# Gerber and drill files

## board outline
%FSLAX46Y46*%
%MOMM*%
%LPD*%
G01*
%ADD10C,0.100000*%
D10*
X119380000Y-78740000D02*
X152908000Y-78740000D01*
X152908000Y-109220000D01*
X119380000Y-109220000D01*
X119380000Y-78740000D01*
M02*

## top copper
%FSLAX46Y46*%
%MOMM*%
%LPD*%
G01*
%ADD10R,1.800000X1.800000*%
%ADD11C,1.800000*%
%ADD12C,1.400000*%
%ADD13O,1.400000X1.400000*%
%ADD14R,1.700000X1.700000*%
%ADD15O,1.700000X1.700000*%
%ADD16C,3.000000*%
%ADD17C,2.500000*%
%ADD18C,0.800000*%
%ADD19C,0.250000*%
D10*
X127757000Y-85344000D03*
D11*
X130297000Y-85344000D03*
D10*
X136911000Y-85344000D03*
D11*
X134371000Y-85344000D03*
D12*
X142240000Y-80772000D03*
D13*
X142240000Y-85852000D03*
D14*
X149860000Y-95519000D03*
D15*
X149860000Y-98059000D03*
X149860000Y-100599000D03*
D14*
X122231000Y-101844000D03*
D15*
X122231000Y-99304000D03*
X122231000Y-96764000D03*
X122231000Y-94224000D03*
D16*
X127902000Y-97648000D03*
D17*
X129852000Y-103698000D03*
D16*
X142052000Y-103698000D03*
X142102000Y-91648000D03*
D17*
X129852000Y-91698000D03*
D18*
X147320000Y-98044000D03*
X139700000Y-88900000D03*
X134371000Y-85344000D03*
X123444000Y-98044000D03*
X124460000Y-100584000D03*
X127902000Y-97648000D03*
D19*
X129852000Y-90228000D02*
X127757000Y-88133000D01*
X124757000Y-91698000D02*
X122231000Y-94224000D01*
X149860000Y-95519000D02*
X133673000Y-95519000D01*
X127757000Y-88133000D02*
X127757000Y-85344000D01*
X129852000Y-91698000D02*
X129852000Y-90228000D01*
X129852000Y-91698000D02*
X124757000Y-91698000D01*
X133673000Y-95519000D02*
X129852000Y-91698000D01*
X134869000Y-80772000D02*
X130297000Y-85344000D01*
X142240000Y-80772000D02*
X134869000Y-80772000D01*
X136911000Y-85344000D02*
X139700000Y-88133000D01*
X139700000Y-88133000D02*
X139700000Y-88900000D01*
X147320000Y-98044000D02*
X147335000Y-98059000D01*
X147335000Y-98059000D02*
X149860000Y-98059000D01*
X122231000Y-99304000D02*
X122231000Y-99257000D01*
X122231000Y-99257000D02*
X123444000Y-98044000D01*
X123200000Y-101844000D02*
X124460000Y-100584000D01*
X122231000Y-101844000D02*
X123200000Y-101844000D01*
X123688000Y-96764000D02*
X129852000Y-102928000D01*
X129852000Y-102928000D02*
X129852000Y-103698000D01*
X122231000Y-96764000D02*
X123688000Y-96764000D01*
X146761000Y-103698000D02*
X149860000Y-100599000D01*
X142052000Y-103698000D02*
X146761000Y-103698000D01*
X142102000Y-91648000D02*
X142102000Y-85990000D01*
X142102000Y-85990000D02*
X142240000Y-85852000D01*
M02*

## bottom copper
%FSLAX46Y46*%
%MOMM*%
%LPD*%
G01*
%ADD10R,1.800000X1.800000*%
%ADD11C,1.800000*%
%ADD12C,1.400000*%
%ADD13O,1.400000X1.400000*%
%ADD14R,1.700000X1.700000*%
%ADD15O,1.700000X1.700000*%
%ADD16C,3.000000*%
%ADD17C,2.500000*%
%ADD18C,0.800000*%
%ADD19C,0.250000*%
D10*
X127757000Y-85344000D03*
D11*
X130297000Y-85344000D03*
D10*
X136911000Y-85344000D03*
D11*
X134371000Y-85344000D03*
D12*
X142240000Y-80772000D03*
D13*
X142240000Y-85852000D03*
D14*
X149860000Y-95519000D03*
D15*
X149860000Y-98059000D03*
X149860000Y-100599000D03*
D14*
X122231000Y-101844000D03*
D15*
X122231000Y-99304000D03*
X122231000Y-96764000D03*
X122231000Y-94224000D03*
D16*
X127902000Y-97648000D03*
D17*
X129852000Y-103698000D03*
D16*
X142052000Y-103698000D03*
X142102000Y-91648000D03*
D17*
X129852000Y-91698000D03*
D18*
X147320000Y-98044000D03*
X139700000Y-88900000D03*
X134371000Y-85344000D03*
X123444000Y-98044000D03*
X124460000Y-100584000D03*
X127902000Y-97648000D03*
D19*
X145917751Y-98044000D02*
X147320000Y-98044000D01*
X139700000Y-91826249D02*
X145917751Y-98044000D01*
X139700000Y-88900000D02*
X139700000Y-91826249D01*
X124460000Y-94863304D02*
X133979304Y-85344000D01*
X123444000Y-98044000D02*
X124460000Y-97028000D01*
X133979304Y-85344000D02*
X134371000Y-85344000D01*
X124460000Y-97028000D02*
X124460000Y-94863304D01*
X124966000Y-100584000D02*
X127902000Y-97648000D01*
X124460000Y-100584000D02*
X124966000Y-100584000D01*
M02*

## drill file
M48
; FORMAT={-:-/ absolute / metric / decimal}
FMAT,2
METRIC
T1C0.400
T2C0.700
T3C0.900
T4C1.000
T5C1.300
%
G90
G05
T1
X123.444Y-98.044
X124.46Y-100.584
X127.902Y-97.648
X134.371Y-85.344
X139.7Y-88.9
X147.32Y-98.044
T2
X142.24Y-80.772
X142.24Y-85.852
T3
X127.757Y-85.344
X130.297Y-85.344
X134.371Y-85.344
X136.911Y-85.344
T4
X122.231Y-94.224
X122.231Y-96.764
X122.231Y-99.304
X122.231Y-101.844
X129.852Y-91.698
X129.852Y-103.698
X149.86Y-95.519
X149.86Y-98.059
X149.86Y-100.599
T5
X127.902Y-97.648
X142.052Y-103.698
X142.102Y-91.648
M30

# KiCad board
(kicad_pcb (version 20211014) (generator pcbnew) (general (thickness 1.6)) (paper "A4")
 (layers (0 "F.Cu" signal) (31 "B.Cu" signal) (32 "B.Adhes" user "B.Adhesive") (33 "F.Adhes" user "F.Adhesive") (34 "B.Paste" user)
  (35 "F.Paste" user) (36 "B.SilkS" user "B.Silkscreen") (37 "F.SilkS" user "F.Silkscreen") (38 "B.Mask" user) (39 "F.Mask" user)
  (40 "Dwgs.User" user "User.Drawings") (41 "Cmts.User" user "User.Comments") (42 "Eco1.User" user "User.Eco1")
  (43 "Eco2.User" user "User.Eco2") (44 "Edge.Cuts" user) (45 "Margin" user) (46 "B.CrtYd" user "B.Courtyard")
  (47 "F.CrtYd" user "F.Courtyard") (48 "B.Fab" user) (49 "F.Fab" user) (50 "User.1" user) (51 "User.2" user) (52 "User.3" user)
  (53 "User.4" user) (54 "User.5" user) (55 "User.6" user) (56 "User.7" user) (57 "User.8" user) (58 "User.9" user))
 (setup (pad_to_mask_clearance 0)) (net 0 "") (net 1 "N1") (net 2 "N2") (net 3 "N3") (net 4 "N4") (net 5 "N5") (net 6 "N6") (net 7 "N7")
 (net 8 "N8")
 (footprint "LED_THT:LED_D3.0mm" (layer "F.Cu") (at 127.757 85.344)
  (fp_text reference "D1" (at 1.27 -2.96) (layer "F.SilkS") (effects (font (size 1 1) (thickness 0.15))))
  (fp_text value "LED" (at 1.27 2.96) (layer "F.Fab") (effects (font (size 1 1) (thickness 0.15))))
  (pad "1" thru_hole rect (at 0 0) (size 1.8 1.8) (drill 0.9) (layers *.Cu *.Mask) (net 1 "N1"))
  (pad "2" thru_hole circle (at 2.54 0) (size 1.8 1.8) (drill 0.9) (layers *.Cu *.Mask) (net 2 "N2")))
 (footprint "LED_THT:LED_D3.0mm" (layer "F.Cu") (at 136.911 85.344 180)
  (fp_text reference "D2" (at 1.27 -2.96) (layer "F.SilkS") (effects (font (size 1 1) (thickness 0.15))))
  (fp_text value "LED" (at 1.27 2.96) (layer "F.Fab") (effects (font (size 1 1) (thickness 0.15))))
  (pad "1" thru_hole rect (at 0 0 180) (size 1.8 1.8) (drill 0.9) (layers *.Cu *.Mask) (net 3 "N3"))
  (pad "2" thru_hole circle (at 2.54 0 180) (size 1.8 1.8) (drill 0.9) (layers *.Cu *.Mask) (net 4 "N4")))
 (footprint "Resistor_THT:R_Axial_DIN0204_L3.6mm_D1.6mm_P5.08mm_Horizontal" (layer "F.Cu") (at 142.24 80.772 -90)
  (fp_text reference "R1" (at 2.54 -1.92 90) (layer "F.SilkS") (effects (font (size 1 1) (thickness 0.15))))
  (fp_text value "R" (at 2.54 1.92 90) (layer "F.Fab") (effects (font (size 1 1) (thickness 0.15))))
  (pad "1" thru_hole circle (at 0 0 270) (size 1.4 1.4) (drill 0.7) (layers *.Cu *.Mask) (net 2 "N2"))
  (pad "2" thru_hole oval (at 5.08 0 270) (size 1.4 1.4) (drill 0.7) (layers *.Cu *.Mask) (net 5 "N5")))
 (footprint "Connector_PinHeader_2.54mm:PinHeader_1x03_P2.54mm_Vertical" (layer "F.Cu") (at 149.86 95.519)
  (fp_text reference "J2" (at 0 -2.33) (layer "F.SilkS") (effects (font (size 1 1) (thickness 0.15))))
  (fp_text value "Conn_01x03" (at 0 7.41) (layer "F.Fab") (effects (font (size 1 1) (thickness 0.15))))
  (pad "1" thru_hole rect (at 0 0) (size 1.7 1.7) (drill 1) (layers *.Cu *.Mask) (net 1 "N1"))
  (pad "2" thru_hole oval (at 0 2.54) (size 1.7 1.7) (drill 1) (layers *.Cu *.Mask) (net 3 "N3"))
  (pad "3" thru_hole oval (at 0 5.08) (size 1.7 1.7) (drill 1) (layers *.Cu *.Mask) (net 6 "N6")))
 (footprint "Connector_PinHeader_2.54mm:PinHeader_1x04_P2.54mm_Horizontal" (layer "F.Cu") (at 122.231 101.844 180)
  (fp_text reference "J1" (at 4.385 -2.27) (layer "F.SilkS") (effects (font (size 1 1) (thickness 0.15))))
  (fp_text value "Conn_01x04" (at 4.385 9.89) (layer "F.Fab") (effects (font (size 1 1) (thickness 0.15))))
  (pad "1" thru_hole rect (at 0 0 180) (size 1.7 1.7) (drill 1) (layers *.Cu *.Mask) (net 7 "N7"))
  (pad "2" thru_hole oval (at 0 2.54 180) (size 1.7 1.7) (drill 1) (layers *.Cu *.Mask) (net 4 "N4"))
  (pad "3" thru_hole oval (at 0 5.08 180) (size 1.7 1.7) (drill 1) (layers *.Cu *.Mask) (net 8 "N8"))
  (pad "4" thru_hole oval (at 0 7.62 180) (size 1.7 1.7) (drill 1) (layers *.Cu *.Mask) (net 1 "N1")))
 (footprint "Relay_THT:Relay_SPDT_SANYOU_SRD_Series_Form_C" (layer "F.Cu") (at 127.902 97.648)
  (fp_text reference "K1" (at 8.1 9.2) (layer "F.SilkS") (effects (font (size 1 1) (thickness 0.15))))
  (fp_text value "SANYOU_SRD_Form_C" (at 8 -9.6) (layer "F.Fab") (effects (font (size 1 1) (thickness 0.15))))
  (pad "1" thru_hole circle (at 0 0 90) (size 3 3) (drill 1.3) (layers *.Cu *.Mask) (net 7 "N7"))
  (pad "2" thru_hole circle (at 1.95 6.05 90) (size 2.5 2.5) (drill 1) (layers *.Cu *.Mask) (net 8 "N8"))
  (pad "3" thru_hole circle (at 14.15 6.05 90) (size 3 3) (drill 1.3) (layers *.Cu *.Mask) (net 6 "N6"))
  (pad "4" thru_hole circle (at 14.2 -6 90) (size 3 3) (drill 1.3) (layers *.Cu *.Mask) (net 5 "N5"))
  (pad "5" thru_hole circle (at 1.95 -5.95 90) (size 2.5 2.5) (drill 1) (layers *.Cu *.Mask) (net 1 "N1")))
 (gr_rect (start 119.38 109.22) (end 152.908 78.74) (layer "Edge.Cuts") (width 0.1) (fill none))
 (segment (start 129.852 90.228) (end 127.757 88.133) (width 0.25) (layer "F.Cu") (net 1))
 (segment (start 124.757 91.698) (end 122.231 94.224) (width 0.25) (layer "F.Cu") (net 1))
 (segment (start 149.86 95.519) (end 133.673 95.519) (width 0.25) (layer "F.Cu") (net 1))
 (segment (start 127.757 88.133) (end 127.757 85.344) (width 0.25) (layer "F.Cu") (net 1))
 (segment (start 129.852 91.698) (end 129.852 90.228) (width 0.25) (layer "F.Cu") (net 1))
 (segment (start 129.852 91.698) (end 124.757 91.698) (width 0.25) (layer "F.Cu") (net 1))
 (segment (start 133.673 95.519) (end 129.852 91.698) (width 0.25) (layer "F.Cu") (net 1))
 (segment (start 134.869 80.772) (end 130.297 85.344) (width 0.25) (layer "F.Cu") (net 2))
 (segment (start 142.24 80.772) (end 134.869 80.772) (width 0.25) (layer "F.Cu") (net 2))
 (segment (start 136.911 85.344) (end 139.7 88.133) (width 0.25) (layer "F.Cu") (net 3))
 (segment (start 139.7 88.133) (end 139.7 88.9) (width 0.25) (layer "F.Cu") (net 3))
 (segment (start 147.32 98.044) (end 147.335 98.059) (width 0.25) (layer "F.Cu") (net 3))
 (segment (start 147.335 98.059) (end 149.86 98.059) (width 0.25) (layer "F.Cu") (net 3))
 (via (at 147.32 98.044) (size 0.8) (drill 0.4) (layers "F.Cu" "B.Cu") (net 3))
 (via (at 139.7 88.9) (size 0.8) (drill 0.4) (layers "F.Cu" "B.Cu") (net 3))
 (segment (start 145.917751 98.044) (end 147.32 98.044) (width 0.25) (layer "B.Cu") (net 3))
 (segment (start 139.7 91.826249) (end 145.917751 98.044) (width 0.25) (layer "B.Cu") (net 3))
 (segment (start 139.7 88.9) (end 139.7 91.826249) (width 0.25) (layer "B.Cu") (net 3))
 (segment (start 122.231 99.304) (end 122.231 99.257) (width 0.25) (layer "F.Cu") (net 4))
 (segment (start 122.231 99.257) (end 123.444 98.044) (width 0.25) (layer "F.Cu") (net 4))
 (via (at 134.371 85.344) (size 0.8) (drill 0.4) (layers "F.Cu" "B.Cu") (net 4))
 (via (at 123.444 98.044) (size 0.8) (drill 0.4) (layers "F.Cu" "B.Cu") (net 4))
 (segment (start 124.46 94.863304) (end 133.979304 85.344) (width 0.25) (layer "B.Cu") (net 4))
 (segment (start 123.444 98.044) (end 124.46 97.028) (width 0.25) (layer "B.Cu") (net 4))
 (segment (start 133.979304 85.344) (end 134.371 85.344) (width 0.25) (layer "B.Cu") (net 4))
 (segment (start 124.46 97.028) (end 124.46 94.863304) (width 0.25) (layer "B.Cu") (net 4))
 (segment (start 123.2 101.844) (end 124.46 100.584) (width 0.25) (layer "F.Cu") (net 7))
 (segment (start 122.231 101.844) (end 123.2 101.844) (width 0.25) (layer "F.Cu") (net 7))
 (via (at 124.46 100.584) (size 0.8) (drill 0.4) (layers "F.Cu" "B.Cu") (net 7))
 (via (at 127.902 97.648) (size 0.8) (drill 0.4) (layers "F.Cu" "B.Cu") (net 7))
 (segment (start 124.966 100.584) (end 127.902 97.648) (width 0.25) (layer "B.Cu") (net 7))
 (segment (start 124.46 100.584) (end 124.966 100.584) (width 0.25) (layer "B.Cu") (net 7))
 (segment (start 123.688 96.764) (end 129.852 102.928) (width 0.25) (layer "F.Cu") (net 8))
 (segment (start 129.852 102.928) (end 129.852 103.698) (width 0.25) (layer "F.Cu") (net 8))
 (segment (start 122.231 96.764) (end 123.688 96.764) (width 0.25) (layer "F.Cu") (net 8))
 (segment (start 146.761 103.698) (end 149.86 100.599) (width 0.25) (layer "F.Cu") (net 6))
 (segment (start 142.052 103.698) (end 146.761 103.698) (width 0.25) (layer "F.Cu") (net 6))
 (segment (start 142.102 91.648) (end 142.102 85.99) (width 0.25) (layer "F.Cu") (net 5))
 (segment (start 142.102 85.99) (end 142.24 85.852) (width 0.25) (layer "F.Cu") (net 5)))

